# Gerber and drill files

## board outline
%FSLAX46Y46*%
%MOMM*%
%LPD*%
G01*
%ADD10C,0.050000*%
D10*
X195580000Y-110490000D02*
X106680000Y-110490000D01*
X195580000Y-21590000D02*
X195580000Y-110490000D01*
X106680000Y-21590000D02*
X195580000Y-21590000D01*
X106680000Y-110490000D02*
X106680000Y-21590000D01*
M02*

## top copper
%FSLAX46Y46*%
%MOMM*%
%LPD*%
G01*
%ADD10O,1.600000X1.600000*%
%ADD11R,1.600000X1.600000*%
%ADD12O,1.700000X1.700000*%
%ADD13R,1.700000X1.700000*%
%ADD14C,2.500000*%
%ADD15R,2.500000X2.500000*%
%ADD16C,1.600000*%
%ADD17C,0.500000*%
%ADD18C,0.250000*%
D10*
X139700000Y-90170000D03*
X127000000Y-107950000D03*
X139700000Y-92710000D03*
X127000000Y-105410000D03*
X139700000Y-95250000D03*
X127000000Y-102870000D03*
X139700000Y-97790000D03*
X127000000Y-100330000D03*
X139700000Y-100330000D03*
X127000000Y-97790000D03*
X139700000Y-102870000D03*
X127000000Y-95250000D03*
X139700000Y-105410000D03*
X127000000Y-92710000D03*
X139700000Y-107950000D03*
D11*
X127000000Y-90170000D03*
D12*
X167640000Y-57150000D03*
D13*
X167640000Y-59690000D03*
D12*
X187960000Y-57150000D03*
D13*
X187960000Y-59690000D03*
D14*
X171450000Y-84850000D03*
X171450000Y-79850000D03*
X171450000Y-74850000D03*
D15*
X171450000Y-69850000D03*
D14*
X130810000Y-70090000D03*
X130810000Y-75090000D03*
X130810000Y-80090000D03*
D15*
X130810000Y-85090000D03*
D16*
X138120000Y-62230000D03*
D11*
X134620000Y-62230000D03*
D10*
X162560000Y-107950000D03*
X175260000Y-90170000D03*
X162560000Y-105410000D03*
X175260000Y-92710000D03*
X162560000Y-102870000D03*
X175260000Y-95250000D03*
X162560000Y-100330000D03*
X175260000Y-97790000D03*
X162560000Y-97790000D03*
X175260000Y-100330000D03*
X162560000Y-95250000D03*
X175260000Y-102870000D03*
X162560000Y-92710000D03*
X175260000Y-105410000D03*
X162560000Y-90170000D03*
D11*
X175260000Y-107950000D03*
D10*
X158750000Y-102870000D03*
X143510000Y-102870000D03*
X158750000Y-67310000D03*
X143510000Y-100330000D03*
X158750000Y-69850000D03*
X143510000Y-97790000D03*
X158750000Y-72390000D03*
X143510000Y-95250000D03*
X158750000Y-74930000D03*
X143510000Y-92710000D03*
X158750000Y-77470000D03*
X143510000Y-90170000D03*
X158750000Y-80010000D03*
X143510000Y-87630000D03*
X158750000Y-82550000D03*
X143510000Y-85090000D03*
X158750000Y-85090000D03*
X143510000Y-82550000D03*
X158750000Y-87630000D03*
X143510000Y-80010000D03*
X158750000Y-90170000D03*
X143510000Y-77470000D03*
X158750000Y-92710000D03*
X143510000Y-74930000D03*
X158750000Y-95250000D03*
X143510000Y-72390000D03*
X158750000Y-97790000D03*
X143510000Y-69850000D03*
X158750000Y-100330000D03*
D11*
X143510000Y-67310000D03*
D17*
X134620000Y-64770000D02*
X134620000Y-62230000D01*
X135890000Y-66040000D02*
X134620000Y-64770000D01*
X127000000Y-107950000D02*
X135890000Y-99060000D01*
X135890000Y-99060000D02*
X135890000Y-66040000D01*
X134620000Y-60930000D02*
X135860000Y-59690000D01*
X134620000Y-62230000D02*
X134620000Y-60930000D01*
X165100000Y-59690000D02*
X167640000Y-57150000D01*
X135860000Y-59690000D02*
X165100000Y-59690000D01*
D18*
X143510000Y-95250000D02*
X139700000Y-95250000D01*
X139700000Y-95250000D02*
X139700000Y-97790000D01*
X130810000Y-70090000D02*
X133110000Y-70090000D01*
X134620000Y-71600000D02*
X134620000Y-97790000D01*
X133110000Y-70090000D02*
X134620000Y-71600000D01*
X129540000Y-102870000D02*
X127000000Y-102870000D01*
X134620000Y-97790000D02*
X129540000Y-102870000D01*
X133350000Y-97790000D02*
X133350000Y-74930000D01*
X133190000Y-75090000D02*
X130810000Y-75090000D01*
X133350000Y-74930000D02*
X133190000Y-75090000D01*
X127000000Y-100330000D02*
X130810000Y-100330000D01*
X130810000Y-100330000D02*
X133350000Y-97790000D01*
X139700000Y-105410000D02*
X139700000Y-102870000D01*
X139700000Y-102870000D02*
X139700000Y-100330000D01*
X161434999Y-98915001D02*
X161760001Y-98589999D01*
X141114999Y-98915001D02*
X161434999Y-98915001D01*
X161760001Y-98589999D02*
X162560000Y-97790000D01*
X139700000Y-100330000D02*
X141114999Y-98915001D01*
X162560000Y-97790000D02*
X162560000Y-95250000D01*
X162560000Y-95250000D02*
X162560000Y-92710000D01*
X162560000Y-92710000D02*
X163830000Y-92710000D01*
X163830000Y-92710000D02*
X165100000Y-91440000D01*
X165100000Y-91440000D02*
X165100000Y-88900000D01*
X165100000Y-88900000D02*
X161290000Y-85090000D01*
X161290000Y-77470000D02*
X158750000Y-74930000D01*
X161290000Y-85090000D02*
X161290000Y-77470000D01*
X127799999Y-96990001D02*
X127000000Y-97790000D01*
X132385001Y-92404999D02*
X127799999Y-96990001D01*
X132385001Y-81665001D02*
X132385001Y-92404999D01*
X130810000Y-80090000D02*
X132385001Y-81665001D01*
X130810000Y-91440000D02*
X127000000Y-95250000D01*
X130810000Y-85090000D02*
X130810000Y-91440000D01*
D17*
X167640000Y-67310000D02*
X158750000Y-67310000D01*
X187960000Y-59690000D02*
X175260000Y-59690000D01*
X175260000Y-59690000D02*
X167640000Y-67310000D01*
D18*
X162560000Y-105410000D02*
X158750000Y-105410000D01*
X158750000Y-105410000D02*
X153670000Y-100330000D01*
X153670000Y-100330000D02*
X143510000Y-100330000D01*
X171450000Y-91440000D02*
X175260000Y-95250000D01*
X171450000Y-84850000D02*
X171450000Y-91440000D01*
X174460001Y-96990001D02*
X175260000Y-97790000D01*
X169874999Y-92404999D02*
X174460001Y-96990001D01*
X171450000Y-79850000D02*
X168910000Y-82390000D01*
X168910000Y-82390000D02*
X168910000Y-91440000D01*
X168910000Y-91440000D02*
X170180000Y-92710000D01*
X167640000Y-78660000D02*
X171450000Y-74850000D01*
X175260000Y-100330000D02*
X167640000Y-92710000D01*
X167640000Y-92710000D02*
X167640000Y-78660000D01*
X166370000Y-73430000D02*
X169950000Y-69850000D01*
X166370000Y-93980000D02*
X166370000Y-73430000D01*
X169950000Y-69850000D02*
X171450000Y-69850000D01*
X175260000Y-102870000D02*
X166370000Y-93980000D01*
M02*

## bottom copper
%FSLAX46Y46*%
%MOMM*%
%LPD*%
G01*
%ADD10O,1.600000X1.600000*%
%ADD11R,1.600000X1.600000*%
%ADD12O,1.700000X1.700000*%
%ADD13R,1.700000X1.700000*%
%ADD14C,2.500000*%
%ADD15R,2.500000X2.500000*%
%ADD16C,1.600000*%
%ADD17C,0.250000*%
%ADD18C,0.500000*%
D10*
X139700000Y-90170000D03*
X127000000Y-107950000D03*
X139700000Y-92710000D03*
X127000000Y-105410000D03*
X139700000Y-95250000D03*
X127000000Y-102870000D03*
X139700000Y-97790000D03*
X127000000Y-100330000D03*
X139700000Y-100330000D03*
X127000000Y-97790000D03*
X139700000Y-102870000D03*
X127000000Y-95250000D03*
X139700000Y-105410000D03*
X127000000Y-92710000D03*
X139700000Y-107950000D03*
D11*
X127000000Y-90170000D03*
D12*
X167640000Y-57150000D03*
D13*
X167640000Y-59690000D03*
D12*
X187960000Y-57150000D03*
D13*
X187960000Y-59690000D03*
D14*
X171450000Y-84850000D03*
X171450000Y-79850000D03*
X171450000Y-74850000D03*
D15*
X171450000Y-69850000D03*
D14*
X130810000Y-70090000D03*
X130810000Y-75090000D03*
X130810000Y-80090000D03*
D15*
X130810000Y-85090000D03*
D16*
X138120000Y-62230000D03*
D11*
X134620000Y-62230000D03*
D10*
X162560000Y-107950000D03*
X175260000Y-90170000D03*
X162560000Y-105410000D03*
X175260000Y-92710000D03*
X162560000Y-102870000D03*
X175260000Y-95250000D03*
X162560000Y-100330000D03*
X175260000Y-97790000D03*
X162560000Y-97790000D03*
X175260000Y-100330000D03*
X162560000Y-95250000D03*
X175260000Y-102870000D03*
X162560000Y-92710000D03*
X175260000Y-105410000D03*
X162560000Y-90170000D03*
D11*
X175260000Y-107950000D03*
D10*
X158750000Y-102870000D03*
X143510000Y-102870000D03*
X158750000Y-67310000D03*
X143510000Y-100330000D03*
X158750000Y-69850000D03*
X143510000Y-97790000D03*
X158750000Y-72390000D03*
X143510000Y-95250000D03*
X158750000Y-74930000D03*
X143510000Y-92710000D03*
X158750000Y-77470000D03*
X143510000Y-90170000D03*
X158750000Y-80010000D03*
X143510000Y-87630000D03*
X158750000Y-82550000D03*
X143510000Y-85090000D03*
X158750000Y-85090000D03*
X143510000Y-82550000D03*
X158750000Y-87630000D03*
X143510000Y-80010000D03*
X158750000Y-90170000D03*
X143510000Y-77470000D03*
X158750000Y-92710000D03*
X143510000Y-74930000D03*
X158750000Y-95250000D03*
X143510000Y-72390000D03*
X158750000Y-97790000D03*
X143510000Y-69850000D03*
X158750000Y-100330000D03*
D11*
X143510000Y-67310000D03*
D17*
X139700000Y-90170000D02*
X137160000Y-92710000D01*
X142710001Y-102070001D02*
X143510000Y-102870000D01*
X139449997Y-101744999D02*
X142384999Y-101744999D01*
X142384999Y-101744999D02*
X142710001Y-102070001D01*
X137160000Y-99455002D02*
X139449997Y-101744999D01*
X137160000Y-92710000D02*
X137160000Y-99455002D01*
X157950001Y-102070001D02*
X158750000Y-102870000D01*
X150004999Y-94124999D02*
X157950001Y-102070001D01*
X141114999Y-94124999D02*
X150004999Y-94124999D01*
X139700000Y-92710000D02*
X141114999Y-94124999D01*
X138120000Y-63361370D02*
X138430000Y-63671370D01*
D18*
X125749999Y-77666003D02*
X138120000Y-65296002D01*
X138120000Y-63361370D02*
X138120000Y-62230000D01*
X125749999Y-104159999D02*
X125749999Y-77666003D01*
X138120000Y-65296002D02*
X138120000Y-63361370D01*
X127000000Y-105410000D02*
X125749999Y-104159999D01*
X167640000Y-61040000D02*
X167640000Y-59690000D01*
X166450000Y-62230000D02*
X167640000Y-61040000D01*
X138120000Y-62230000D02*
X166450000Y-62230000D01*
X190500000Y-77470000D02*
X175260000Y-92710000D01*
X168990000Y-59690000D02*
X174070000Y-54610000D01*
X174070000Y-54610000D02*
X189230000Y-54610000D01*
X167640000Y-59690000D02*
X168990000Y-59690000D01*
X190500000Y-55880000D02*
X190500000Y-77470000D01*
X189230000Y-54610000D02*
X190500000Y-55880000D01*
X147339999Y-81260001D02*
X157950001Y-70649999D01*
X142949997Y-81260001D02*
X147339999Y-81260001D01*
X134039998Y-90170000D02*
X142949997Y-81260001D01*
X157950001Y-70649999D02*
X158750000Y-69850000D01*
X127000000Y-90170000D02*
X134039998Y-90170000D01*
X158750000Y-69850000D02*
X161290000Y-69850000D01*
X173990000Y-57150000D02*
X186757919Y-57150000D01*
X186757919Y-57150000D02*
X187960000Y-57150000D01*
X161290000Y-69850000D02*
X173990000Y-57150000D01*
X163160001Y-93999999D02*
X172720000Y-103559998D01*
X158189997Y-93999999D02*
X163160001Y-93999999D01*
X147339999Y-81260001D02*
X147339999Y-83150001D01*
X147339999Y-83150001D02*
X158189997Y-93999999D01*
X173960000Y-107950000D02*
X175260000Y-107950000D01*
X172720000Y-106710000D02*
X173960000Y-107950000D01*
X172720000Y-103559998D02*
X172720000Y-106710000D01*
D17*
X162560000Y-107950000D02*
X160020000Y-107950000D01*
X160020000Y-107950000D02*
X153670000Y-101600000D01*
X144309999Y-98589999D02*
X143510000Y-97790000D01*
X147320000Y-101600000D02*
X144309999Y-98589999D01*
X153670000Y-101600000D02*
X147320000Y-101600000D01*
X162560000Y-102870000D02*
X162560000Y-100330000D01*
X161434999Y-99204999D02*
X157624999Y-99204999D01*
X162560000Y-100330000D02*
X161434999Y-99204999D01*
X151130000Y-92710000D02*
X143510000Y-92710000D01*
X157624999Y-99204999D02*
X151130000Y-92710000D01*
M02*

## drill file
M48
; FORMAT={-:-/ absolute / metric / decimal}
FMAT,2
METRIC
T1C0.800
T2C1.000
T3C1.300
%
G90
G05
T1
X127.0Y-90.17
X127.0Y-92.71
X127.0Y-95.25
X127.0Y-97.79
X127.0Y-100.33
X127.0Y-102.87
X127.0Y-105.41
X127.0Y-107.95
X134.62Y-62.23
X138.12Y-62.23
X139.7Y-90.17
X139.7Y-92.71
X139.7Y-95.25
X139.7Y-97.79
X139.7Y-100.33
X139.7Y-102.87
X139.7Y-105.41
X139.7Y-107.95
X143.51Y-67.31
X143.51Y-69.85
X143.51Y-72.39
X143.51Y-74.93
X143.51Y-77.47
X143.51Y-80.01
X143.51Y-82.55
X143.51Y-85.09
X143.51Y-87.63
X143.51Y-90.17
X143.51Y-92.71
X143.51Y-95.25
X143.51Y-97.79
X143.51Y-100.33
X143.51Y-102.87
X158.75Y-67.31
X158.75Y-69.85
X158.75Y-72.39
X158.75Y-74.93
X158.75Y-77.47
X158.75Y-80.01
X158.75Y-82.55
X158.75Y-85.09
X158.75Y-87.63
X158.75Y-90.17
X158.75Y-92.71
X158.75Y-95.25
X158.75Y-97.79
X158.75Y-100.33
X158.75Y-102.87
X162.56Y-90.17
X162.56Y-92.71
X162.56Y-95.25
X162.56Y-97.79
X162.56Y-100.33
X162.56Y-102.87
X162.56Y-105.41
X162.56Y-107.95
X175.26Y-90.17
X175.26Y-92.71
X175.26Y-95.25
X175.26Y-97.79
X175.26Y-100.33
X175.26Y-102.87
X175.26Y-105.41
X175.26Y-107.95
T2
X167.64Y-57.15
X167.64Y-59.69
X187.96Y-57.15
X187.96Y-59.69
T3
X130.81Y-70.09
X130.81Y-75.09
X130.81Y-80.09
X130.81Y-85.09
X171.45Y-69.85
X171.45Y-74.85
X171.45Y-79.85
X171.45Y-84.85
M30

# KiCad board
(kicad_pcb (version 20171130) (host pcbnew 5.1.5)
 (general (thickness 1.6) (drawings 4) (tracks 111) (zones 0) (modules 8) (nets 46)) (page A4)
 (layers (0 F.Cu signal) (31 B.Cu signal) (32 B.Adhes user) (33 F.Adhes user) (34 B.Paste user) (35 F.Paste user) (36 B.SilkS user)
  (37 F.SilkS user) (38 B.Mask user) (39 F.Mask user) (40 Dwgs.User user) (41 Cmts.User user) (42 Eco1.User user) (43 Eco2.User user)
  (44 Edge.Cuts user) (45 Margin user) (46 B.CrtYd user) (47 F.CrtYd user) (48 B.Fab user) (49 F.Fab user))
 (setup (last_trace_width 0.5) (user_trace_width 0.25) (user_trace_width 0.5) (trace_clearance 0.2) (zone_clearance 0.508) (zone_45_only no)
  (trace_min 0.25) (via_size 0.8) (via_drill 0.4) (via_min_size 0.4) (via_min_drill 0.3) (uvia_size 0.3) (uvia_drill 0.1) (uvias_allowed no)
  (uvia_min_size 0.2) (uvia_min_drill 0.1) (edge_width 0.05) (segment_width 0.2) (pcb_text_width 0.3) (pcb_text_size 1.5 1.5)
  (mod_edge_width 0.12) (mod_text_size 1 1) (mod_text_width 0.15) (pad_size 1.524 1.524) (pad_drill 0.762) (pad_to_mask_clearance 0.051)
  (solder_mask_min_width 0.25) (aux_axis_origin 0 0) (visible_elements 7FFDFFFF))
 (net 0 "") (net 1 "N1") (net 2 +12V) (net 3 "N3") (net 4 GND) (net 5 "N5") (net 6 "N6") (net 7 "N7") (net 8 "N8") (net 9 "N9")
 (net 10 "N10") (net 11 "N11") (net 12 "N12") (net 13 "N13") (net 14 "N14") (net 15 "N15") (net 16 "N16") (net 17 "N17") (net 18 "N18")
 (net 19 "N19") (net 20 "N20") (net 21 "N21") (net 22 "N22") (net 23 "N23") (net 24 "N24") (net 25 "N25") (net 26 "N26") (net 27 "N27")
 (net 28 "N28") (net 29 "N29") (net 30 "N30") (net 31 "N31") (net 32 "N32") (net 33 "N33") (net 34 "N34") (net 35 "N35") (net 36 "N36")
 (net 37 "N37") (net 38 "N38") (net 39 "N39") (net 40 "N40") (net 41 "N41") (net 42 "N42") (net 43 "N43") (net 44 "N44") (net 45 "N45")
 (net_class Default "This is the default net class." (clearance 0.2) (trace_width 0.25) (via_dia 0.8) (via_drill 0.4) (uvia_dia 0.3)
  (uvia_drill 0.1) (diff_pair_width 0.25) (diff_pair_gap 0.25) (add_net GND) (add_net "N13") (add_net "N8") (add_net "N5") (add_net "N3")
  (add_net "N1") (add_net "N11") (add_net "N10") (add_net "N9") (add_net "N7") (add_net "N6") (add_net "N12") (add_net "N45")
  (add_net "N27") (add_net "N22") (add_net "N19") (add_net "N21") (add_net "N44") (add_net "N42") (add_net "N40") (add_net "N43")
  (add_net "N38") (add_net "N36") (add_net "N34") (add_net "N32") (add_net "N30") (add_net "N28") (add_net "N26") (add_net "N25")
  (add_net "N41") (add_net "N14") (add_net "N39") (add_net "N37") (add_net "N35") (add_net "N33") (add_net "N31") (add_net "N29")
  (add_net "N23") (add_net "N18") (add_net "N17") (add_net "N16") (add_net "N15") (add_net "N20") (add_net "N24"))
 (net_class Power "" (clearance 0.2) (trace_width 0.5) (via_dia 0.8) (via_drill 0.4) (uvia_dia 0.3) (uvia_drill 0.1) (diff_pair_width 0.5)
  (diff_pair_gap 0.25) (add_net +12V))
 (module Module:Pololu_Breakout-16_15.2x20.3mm (layer F.Cu) (at 127 90.17)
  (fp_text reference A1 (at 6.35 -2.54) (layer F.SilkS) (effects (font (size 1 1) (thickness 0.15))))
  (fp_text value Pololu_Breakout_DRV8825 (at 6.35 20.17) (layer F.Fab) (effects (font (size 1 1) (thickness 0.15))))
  (pad 16 thru_hole oval (at 12.7 0) (size 1.6 1.6) (drill 0.8) (layers *.Cu *.Mask) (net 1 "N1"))
  (pad 8 thru_hole oval (at 0 17.78) (size 1.6 1.6) (drill 0.8) (layers *.Cu *.Mask) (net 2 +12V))
  (pad 15 thru_hole oval (at 12.7 2.54) (size 1.6 1.6) (drill 0.8) (layers *.Cu *.Mask) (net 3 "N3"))
  (pad 7 thru_hole oval (at 0 15.24) (size 1.6 1.6) (drill 0.8) (layers *.Cu *.Mask) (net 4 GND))
  (pad 14 thru_hole oval (at 12.7 5.08) (size 1.6 1.6) (drill 0.8) (layers *.Cu *.Mask) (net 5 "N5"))
  (pad 6 thru_hole oval (at 0 12.7) (size 1.6 1.6) (drill 0.8) (layers *.Cu *.Mask) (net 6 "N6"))
  (pad 13 thru_hole oval (at 12.7 7.62) (size 1.6 1.6) (drill 0.8) (layers *.Cu *.Mask) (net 5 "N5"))
  (pad 5 thru_hole oval (at 0 10.16) (size 1.6 1.6) (drill 0.8) (layers *.Cu *.Mask) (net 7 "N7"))
  (pad 12 thru_hole oval (at 12.7 10.16) (size 1.6 1.6) (drill 0.8) (layers *.Cu *.Mask) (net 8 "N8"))
  (pad 4 thru_hole oval (at 0 7.62) (size 1.6 1.6) (drill 0.8) (layers *.Cu *.Mask) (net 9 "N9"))
  (pad 11 thru_hole oval (at 12.7 12.7) (size 1.6 1.6) (drill 0.8) (layers *.Cu *.Mask) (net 8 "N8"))
  (pad 3 thru_hole oval (at 0 5.08) (size 1.6 1.6) (drill 0.8) (layers *.Cu *.Mask) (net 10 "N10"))
  (pad 10 thru_hole oval (at 12.7 15.24) (size 1.6 1.6) (drill 0.8) (layers *.Cu *.Mask) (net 8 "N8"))
  (pad 2 thru_hole oval (at 0 2.54) (size 1.6 1.6) (drill 0.8) (layers *.Cu *.Mask) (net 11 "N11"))
  (pad 9 thru_hole oval (at 12.7 17.78) (size 1.6 1.6) (drill 0.8) (layers *.Cu *.Mask) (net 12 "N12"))
  (pad 1 thru_hole rect (at 0 0) (size 1.6 1.6) (drill 0.8) (layers *.Cu *.Mask) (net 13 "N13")))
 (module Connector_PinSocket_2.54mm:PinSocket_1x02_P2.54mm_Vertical (layer F.Cu) (at 167.64 59.69 180)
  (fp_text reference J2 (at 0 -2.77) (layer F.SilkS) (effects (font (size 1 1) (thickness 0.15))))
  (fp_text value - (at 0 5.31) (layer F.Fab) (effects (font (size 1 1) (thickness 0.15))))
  (pad 2 thru_hole oval (at 0 2.54 180) (size 1.7 1.7) (drill 1) (layers *.Cu *.Mask) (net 2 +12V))
  (pad 1 thru_hole rect (at 0 0 180) (size 1.7 1.7) (drill 1) (layers *.Cu *.Mask) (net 4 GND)))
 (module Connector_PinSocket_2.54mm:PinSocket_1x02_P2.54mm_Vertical (layer F.Cu) (at 187.96 59.69 180)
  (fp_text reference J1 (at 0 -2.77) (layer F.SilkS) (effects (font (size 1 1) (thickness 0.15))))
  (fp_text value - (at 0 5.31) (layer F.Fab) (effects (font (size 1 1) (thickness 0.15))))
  (pad 2 thru_hole oval (at 0 2.54 180) (size 1.7 1.7) (drill 1) (layers *.Cu *.Mask) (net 13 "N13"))
  (pad 1 thru_hole rect (at 0 0 180) (size 1.7 1.7) (drill 1) (layers *.Cu *.Mask) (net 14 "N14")))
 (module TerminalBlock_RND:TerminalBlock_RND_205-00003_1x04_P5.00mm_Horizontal (layer F.Cu) (at 171.45 69.85 270)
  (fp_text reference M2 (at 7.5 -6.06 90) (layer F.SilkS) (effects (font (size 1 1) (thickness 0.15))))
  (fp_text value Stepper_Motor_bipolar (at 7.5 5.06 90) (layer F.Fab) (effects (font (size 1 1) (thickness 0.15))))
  (pad 4 thru_hole circle (at 15 0 270) (size 2.5 2.5) (drill 1.3) (layers *.Cu *.Mask) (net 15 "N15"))
  (pad 3 thru_hole circle (at 10 0 270) (size 2.5 2.5) (drill 1.3) (layers *.Cu *.Mask) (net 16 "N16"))
  (pad 2 thru_hole circle (at 5 0 270) (size 2.5 2.5) (drill 1.3) (layers *.Cu *.Mask) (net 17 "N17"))
  (pad 1 thru_hole rect (at 0 0 270) (size 2.5 2.5) (drill 1.3) (layers *.Cu *.Mask) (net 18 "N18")))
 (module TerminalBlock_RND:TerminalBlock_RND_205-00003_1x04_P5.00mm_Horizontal (layer F.Cu) (at 130.81 85.09 90)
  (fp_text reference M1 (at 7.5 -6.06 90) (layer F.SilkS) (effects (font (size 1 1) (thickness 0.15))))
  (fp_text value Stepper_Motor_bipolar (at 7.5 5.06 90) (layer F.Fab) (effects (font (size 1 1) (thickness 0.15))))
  (pad 4 thru_hole circle (at 15 0 90) (size 2.5 2.5) (drill 1.3) (layers *.Cu *.Mask) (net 6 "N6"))
  (pad 3 thru_hole circle (at 10 0 90) (size 2.5 2.5) (drill 1.3) (layers *.Cu *.Mask) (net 7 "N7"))
  (pad 2 thru_hole circle (at 5 0 90) (size 2.5 2.5) (drill 1.3) (layers *.Cu *.Mask) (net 9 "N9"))
  (pad 1 thru_hole rect (at 0 0 90) (size 2.5 2.5) (drill 1.3) (layers *.Cu *.Mask) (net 10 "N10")))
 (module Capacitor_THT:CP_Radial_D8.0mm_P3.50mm (layer F.Cu) (at 134.62 62.23)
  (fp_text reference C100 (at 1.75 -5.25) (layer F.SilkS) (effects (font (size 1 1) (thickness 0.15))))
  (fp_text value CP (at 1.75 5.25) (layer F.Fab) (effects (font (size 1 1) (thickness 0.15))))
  (pad 2 thru_hole circle (at 3.5 0) (size 1.6 1.6) (drill 0.8) (layers *.Cu *.Mask) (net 4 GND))
  (pad 1 thru_hole rect (at 0 0) (size 1.6 1.6) (drill 0.8) (layers *.Cu *.Mask) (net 2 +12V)))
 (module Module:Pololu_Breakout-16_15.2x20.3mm (layer F.Cu) (at 175.26 107.95 180)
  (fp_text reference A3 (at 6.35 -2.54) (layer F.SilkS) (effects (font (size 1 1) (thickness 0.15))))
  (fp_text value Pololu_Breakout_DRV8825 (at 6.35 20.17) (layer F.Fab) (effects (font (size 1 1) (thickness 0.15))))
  (pad 16 thru_hole oval (at 12.7 0 180) (size 1.6 1.6) (drill 0.8) (layers *.Cu *.Mask) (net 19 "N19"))
  (pad 8 thru_hole oval (at 0 17.78 180) (size 1.6 1.6) (drill 0.8) (layers *.Cu *.Mask) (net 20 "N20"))
  (pad 15 thru_hole oval (at 12.7 2.54 180) (size 1.6 1.6) (drill 0.8) (layers *.Cu *.Mask) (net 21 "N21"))
  (pad 7 thru_hole oval (at 0 15.24 180) (size 1.6 1.6) (drill 0.8) (layers *.Cu *.Mask) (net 4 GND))
  (pad 14 thru_hole oval (at 12.7 5.08 180) (size 1.6 1.6) (drill 0.8) (layers *.Cu *.Mask) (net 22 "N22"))
  (pad 6 thru_hole oval (at 0 12.7 180) (size 1.6 1.6) (drill 0.8) (layers *.Cu *.Mask) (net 15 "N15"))
  (pad 13 thru_hole oval (at 12.7 7.62 180) (size 1.6 1.6) (drill 0.8) (layers *.Cu *.Mask) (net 22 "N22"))
  (pad 5 thru_hole oval (at 0 10.16 180) (size 1.6 1.6) (drill 0.8) (layers *.Cu *.Mask) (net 16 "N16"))
  (pad 12 thru_hole oval (at 12.7 10.16 180) (size 1.6 1.6) (drill 0.8) (layers *.Cu *.Mask) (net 8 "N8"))
  (pad 4 thru_hole oval (at 0 7.62 180) (size 1.6 1.6) (drill 0.8) (layers *.Cu *.Mask) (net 17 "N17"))
  (pad 11 thru_hole oval (at 12.7 12.7 180) (size 1.6 1.6) (drill 0.8) (layers *.Cu *.Mask) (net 8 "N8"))
  (pad 3 thru_hole oval (at 0 5.08 180) (size 1.6 1.6) (drill 0.8) (layers *.Cu *.Mask) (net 18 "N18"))
  (pad 10 thru_hole oval (at 12.7 15.24 180) (size 1.6 1.6) (drill 0.8) (layers *.Cu *.Mask) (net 8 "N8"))
  (pad 2 thru_hole oval (at 0 2.54 180) (size 1.6 1.6) (drill 0.8) (layers *.Cu *.Mask) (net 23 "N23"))
  (pad 9 thru_hole oval (at 12.7 17.78 180) (size 1.6 1.6) (drill 0.8) (layers *.Cu *.Mask) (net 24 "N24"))
  (pad 1 thru_hole rect (at 0 0 180) (size 1.6 1.6) (drill 0.8) (layers *.Cu *.Mask) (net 13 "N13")))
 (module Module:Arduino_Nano (layer F.Cu) (at 143.51 67.31)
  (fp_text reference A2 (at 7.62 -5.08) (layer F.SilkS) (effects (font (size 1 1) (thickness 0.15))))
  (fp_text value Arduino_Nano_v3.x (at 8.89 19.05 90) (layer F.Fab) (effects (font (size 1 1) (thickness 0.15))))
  (pad 16 thru_hole oval (at 15.24 35.56) (size 1.6 1.6) (drill 0.8) (layers *.Cu *.Mask) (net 3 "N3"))
  (pad 15 thru_hole oval (at 0 35.56) (size 1.6 1.6) (drill 0.8) (layers *.Cu *.Mask) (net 1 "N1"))
  (pad 30 thru_hole oval (at 15.24 0) (size 1.6 1.6) (drill 0.8) (layers *.Cu *.Mask) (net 14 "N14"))
  (pad 14 thru_hole oval (at 0 33.02) (size 1.6 1.6) (drill 0.8) (layers *.Cu *.Mask) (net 21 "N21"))
  (pad 29 thru_hole oval (at 15.24 2.54) (size 1.6 1.6) (drill 0.8) (layers *.Cu *.Mask) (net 13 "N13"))
  (pad 13 thru_hole oval (at 0 30.48) (size 1.6 1.6) (drill 0.8) (layers *.Cu *.Mask) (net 19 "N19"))
  (pad 28 thru_hole oval (at 15.24 5.08) (size 1.6 1.6) (drill 0.8) (layers *.Cu *.Mask) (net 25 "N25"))
  (pad 12 thru_hole oval (at 0 27.94) (size 1.6 1.6) (drill 0.8) (layers *.Cu *.Mask) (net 5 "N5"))
  (pad 27 thru_hole oval (at 15.24 7.62) (size 1.6 1.6) (drill 0.8) (layers *.Cu *.Mask) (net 8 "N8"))
  (pad 11 thru_hole oval (at 0 25.4) (size 1.6 1.6) (drill 0.8) (layers *.Cu *.Mask) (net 22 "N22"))
  (pad 26 thru_hole oval (at 15.24 10.16) (size 1.6 1.6) (drill 0.8) (layers *.Cu *.Mask) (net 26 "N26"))
  (pad 10 thru_hole oval (at 0 22.86) (size 1.6 1.6) (drill 0.8) (layers *.Cu *.Mask) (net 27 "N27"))
  (pad 25 thru_hole oval (at 15.24 12.7) (size 1.6 1.6) (drill 0.8) (layers *.Cu *.Mask) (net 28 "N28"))
  (pad 9 thru_hole oval (at 0 20.32) (size 1.6 1.6) (drill 0.8) (layers *.Cu *.Mask) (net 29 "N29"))
  (pad 24 thru_hole oval (at 15.24 15.24) (size 1.6 1.6) (drill 0.8) (layers *.Cu *.Mask) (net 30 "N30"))
  (pad 8 thru_hole oval (at 0 17.78) (size 1.6 1.6) (drill 0.8) (layers *.Cu *.Mask) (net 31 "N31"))
  (pad 23 thru_hole oval (at 15.24 17.78) (size 1.6 1.6) (drill 0.8) (layers *.Cu *.Mask) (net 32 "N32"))
  (pad 7 thru_hole oval (at 0 15.24) (size 1.6 1.6) (drill 0.8) (layers *.Cu *.Mask) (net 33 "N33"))
  (pad 22 thru_hole oval (at 15.24 20.32) (size 1.6 1.6) (drill 0.8) (layers *.Cu *.Mask) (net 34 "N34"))
  (pad 6 thru_hole oval (at 0 12.7) (size 1.6 1.6) (drill 0.8) (layers *.Cu *.Mask) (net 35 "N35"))
  (pad 21 thru_hole oval (at 15.24 22.86) (size 1.6 1.6) (drill 0.8) (layers *.Cu *.Mask) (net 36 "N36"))
  (pad 5 thru_hole oval (at 0 10.16) (size 1.6 1.6) (drill 0.8) (layers *.Cu *.Mask) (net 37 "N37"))
  (pad 20 thru_hole oval (at 15.24 25.4) (size 1.6 1.6) (drill 0.8) (layers *.Cu *.Mask) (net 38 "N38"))
  (pad 4 thru_hole oval (at 0 7.62) (size 1.6 1.6) (drill 0.8) (layers *.Cu *.Mask) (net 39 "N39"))
  (pad 19 thru_hole oval (at 15.24 27.94) (size 1.6 1.6) (drill 0.8) (layers *.Cu *.Mask) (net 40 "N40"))
  (pad 3 thru_hole oval (at 0 5.08) (size 1.6 1.6) (drill 0.8) (layers *.Cu *.Mask) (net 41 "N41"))
  (pad 18 thru_hole oval (at 15.24 30.48) (size 1.6 1.6) (drill 0.8) (layers *.Cu *.Mask) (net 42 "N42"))
  (pad 2 thru_hole oval (at 0 2.54) (size 1.6 1.6) (drill 0.8) (layers *.Cu *.Mask) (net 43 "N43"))
  (pad 17 thru_hole oval (at 15.24 33.02) (size 1.6 1.6) (drill 0.8) (layers *.Cu *.Mask) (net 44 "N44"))
  (pad 1 thru_hole rect (at 0 0) (size 1.6 1.6) (drill 0.8) (layers *.Cu *.Mask) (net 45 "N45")))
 (gr_line (start 195.58 110.49) (end 106.68 110.49) (layer Edge.Cuts) (width 0.05))
 (gr_line (start 195.58 21.59) (end 195.58 110.49) (layer Edge.Cuts) (width 0.05))
 (gr_line (start 106.68 21.59) (end 195.58 21.59) (layer Edge.Cuts) (width 0.05))
 (gr_line (start 106.68 110.49) (end 106.68 21.59) (layer Edge.Cuts) (width 0.05))
 (segment (start 139.7 90.17) (end 137.16 92.71) (width 0.25) (layer B.Cu) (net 1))
 (segment (start 142.710001 102.070001) (end 143.51 102.87) (width 0.25) (layer B.Cu) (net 1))
 (segment (start 139.449997 101.744999) (end 142.384999 101.744999) (width 0.25) (layer B.Cu) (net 1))
 (segment (start 142.384999 101.744999) (end 142.710001 102.070001) (width 0.25) (layer B.Cu) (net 1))
 (segment (start 137.16 99.455002) (end 139.449997 101.744999) (width 0.25) (layer B.Cu) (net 1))
 (segment (start 137.16 92.71) (end 137.16 99.455002) (width 0.25) (layer B.Cu) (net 1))
 (segment (start 134.62 64.77) (end 134.62 62.23) (width 0.5) (layer F.Cu) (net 2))
 (segment (start 135.89 66.04) (end 134.62 64.77) (width 0.5) (layer F.Cu) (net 2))
 (segment (start 127 107.95) (end 135.89 99.06) (width 0.5) (layer F.Cu) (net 2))
 (segment (start 135.89 99.06) (end 135.89 66.04) (width 0.5) (layer F.Cu) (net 2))
 (segment (start 134.62 60.93) (end 135.86 59.69) (width 0.5) (layer F.Cu) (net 2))
 (segment (start 134.62 62.23) (end 134.62 60.93) (width 0.5) (layer F.Cu) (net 2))
 (segment (start 165.1 59.69) (end 167.64 57.15) (width 0.5) (layer F.Cu) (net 2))
 (segment (start 135.86 59.69) (end 165.1 59.69) (width 0.5) (layer F.Cu) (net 2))
 (segment (start 157.950001 102.070001) (end 158.75 102.87) (width 0.25) (layer B.Cu) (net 3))
 (segment (start 150.004999 94.124999) (end 157.950001 102.070001) (width 0.25) (layer B.Cu) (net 3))
 (segment (start 141.114999 94.124999) (end 150.004999 94.124999) (width 0.25) (layer B.Cu) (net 3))
 (segment (start 139.7 92.71) (end 141.114999 94.124999) (width 0.25) (layer B.Cu) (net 3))
 (segment (start 138.12 63.36137) (end 138.43 63.67137) (width 0.25) (layer B.Cu) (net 4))
 (segment (start 125.749999 77.666003) (end 138.12 65.296002) (width 0.5) (layer B.Cu) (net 4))
 (segment (start 138.12 63.36137) (end 138.12 62.23) (width 0.5) (layer B.Cu) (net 4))
 (segment (start 125.749999 104.159999) (end 125.749999 77.666003) (width 0.5) (layer B.Cu) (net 4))
 (segment (start 138.12 65.296002) (end 138.12 63.36137) (width 0.5) (layer B.Cu) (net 4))
 (segment (start 127 105.41) (end 125.749999 104.159999) (width 0.5) (layer B.Cu) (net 4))
 (segment (start 167.64 61.04) (end 167.64 59.69) (width 0.5) (layer B.Cu) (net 4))
 (segment (start 166.45 62.23) (end 167.64 61.04) (width 0.5) (layer B.Cu) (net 4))
 (segment (start 138.12 62.23) (end 166.45 62.23) (width 0.5) (layer B.Cu) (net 4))
 (segment (start 190.5 77.47) (end 175.26 92.71) (width 0.5) (layer B.Cu) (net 4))
 (segment (start 168.99 59.69) (end 174.07 54.61) (width 0.5) (layer B.Cu) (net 4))
 (segment (start 174.07 54.61) (end 189.23 54.61) (width 0.5) (layer B.Cu) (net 4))
 (segment (start 167.64 59.69) (end 168.99 59.69) (width 0.5) (layer B.Cu) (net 4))
 (segment (start 190.5 55.88) (end 190.5 77.47) (width 0.5) (layer B.Cu) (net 4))
 (segment (start 189.23 54.61) (end 190.5 55.88) (width 0.5) (layer B.Cu) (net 4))
 (segment (start 143.51 95.25) (end 139.7 95.25) (width 0.25) (layer F.Cu) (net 5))
 (segment (start 139.7 95.25) (end 139.7 97.79) (width 0.25) (layer F.Cu) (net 5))
 (segment (start 130.81 70.09) (end 133.11 70.09) (width 0.25) (layer F.Cu) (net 6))
 (segment (start 134.62 71.6) (end 134.62 97.79) (width 0.25) (layer F.Cu) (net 6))
 (segment (start 133.11 70.09) (end 134.62 71.6) (width 0.25) (layer F.Cu) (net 6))
 (segment (start 129.54 102.87) (end 127 102.87) (width 0.25) (layer F.Cu) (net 6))
 (segment (start 134.62 97.79) (end 129.54 102.87) (width 0.25) (layer F.Cu) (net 6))
 (segment (start 133.35 97.79) (end 133.35 74.93) (width 0.25) (layer F.Cu) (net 7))
 (segment (start 133.19 75.09) (end 130.81 75.09) (width 0.25) (layer F.Cu) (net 7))
 (segment (start 133.35 74.93) (end 133.19 75.09) (width 0.25) (layer F.Cu) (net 7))
 (segment (start 127 100.33) (end 130.81 100.33) (width 0.25) (layer F.Cu) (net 7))
 (segment (start 130.81 100.33) (end 133.35 97.79) (width 0.25) (layer F.Cu) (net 7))
 (segment (start 139.7 105.41) (end 139.7 102.87) (width 0.25) (layer F.Cu) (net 8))
 (segment (start 139.7 102.87) (end 139.7 100.33) (width 0.25) (layer F.Cu) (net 8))
 (segment (start 161.434999 98.915001) (end 161.760001 98.589999) (width 0.25) (layer F.Cu) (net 8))
 (segment (start 141.114999 98.915001) (end 161.434999 98.915001) (width 0.25) (layer F.Cu) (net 8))
 (segment (start 161.760001 98.589999) (end 162.56 97.79) (width 0.25) (layer F.Cu) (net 8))
 (segment (start 139.7 100.33) (end 141.114999 98.915001) (width 0.25) (layer F.Cu) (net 8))
 (segment (start 162.56 97.79) (end 162.56 95.25) (width 0.25) (layer F.Cu) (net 8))
 (segment (start 162.56 95.25) (end 162.56 92.71) (width 0.25) (layer F.Cu) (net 8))
 (segment (start 162.56 92.71) (end 163.83 92.71) (width 0.25) (layer F.Cu) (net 8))
 (segment (start 163.83 92.71) (end 165.1 91.44) (width 0.25) (layer F.Cu) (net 8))
 (segment (start 165.1 91.44) (end 165.1 88.9) (width 0.25) (layer F.Cu) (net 8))
 (segment (start 165.1 88.9) (end 161.29 85.09) (width 0.25) (layer F.Cu) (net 8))
 (segment (start 161.29 77.47) (end 158.75 74.93) (width 0.25) (layer F.Cu) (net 8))
 (segment (start 161.29 85.09) (end 161.29 77.47) (width 0.25) (layer F.Cu) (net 8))
 (segment (start 127.799999 96.990001) (end 127 97.79) (width 0.25) (layer F.Cu) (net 9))
 (segment (start 132.385001 92.404999) (end 127.799999 96.990001) (width 0.25) (layer F.Cu) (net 9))
 (segment (start 132.385001 81.665001) (end 132.385001 92.404999) (width 0.25) (layer F.Cu) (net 9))
 (segment (start 130.81 80.09) (end 132.385001 81.665001) (width 0.25) (layer F.Cu) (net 9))
 (segment (start 130.81 91.44) (end 127 95.25) (width 0.25) (layer F.Cu) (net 10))
 (segment (start 130.81 85.09) (end 130.81 91.44) (width 0.25) (layer F.Cu) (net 10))
 (segment (start 147.339999 81.260001) (end 157.950001 70.649999) (width 0.5) (layer B.Cu) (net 13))
 (segment (start 142.949997 81.260001) (end 147.339999 81.260001) (width 0.5) (layer B.Cu) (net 13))
 (segment (start 134.039998 90.17) (end 142.949997 81.260001) (width 0.5) (layer B.Cu) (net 13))
 (segment (start 157.950001 70.649999) (end 158.75 69.85) (width 0.5) (layer B.Cu) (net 13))
 (segment (start 127 90.17) (end 134.039998 90.17) (width 0.5) (layer B.Cu) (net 13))
 (segment (start 158.75 69.85) (end 161.29 69.85) (width 0.5) (layer B.Cu) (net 13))
 (segment (start 173.99 57.15) (end 186.757919 57.15) (width 0.5) (layer B.Cu) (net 13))
 (segment (start 186.757919 57.15) (end 187.96 57.15) (width 0.5) (layer B.Cu) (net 13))
 (segment (start 161.29 69.85) (end 173.99 57.15) (width 0.5) (layer B.Cu) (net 13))
 (segment (start 163.160001 93.999999) (end 172.72 103.559998) (width 0.5) (layer B.Cu) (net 13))
 (segment (start 158.189997 93.999999) (end 163.160001 93.999999) (width 0.5) (layer B.Cu) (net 13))
 (segment (start 147.339999 81.260001) (end 147.339999 83.150001) (width 0.5) (layer B.Cu) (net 13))
 (segment (start 147.339999 83.150001) (end 158.189997 93.999999) (width 0.5) (layer B.Cu) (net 13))
 (segment (start 173.96 107.95) (end 175.26 107.95) (width 0.5) (layer B.Cu) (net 13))
 (segment (start 172.72 106.71) (end 173.96 107.95) (width 0.5) (layer B.Cu) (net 13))
 (segment (start 172.72 103.559998) (end 172.72 106.71) (width 0.5) (layer B.Cu) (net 13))
 (segment (start 167.64 67.31) (end 158.75 67.31) (width 0.5) (layer F.Cu) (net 14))
 (segment (start 187.96 59.69) (end 175.26 59.69) (width 0.5) (layer F.Cu) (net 14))
 (segment (start 175.26 59.69) (end 167.64 67.31) (width 0.5) (layer F.Cu) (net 14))
 (segment (start 162.56 105.41) (end 158.75 105.41) (width 0.25) (layer F.Cu) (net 21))
 (segment (start 158.75 105.41) (end 153.67 100.33) (width 0.25) (layer F.Cu) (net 21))
 (segment (start 153.67 100.33) (end 143.51 100.33) (width 0.25) (layer F.Cu) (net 21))
 (segment (start 162.56 107.95) (end 160.02 107.95) (width 0.25) (layer B.Cu) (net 19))
 (segment (start 160.02 107.95) (end 153.67 101.6) (width 0.25) (layer B.Cu) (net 19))
 (segment (start 144.309999 98.589999) (end 143.51 97.79) (width 0.25) (layer B.Cu) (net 19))
 (segment (start 147.32 101.6) (end 144.309999 98.589999) (width 0.25) (layer B.Cu) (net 19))
 (segment (start 153.67 101.6) (end 147.32 101.6) (width 0.25) (layer B.Cu) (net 19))
 (segment (start 162.56 102.87) (end 162.56 100.33) (width 0.25) (layer B.Cu) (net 22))
 (segment (start 161.434999 99.204999) (end 157.624999 99.204999) (width 0.25) (layer B.Cu) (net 22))
 (segment (start 162.56 100.33) (end 161.434999 99.204999) (width 0.25) (layer B.Cu) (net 22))
 (segment (start 151.13 92.71) (end 143.51 92.71) (width 0.25) (layer B.Cu) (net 22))
 (segment (start 157.624999 99.204999) (end 151.13 92.71) (width 0.25) (layer B.Cu) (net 22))
 (segment (start 171.45 91.44) (end 175.26 95.25) (width 0.25) (layer F.Cu) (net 15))
 (segment (start 171.45 84.85) (end 171.45 91.44) (width 0.25) (layer F.Cu) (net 15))
 (segment (start 174.460001 96.990001) (end 175.26 97.79) (width 0.25) (layer F.Cu) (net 16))
 (segment (start 169.874999 92.404999) (end 174.460001 96.990001) (width 0.25) (layer F.Cu) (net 16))
 (segment (start 171.45 79.85) (end 168.91 82.39) (width 0.25) (layer F.Cu) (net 16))
 (segment (start 168.91 82.39) (end 168.91 91.44) (width 0.25) (layer F.Cu) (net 16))
 (segment (start 168.91 91.44) (end 170.18 92.71) (width 0.25) (layer F.Cu) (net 16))
 (segment (start 167.64 78.66) (end 171.45 74.85) (width 0.25) (layer F.Cu) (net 17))
 (segment (start 175.26 100.33) (end 167.64 92.71) (width 0.25) (layer F.Cu) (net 17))
 (segment (start 167.64 92.71) (end 167.64 78.66) (width 0.25) (layer F.Cu) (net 17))
 (segment (start 166.37 73.43) (end 169.95 69.85) (width 0.25) (layer F.Cu) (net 18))
 (segment (start 166.37 93.98) (end 166.37 73.43) (width 0.25) (layer F.Cu) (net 18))
 (segment (start 169.95 69.85) (end 171.45 69.85) (width 0.25) (layer F.Cu) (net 18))
 (segment (start 175.26 102.87) (end 166.37 93.98) (width 0.25) (layer F.Cu) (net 18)))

